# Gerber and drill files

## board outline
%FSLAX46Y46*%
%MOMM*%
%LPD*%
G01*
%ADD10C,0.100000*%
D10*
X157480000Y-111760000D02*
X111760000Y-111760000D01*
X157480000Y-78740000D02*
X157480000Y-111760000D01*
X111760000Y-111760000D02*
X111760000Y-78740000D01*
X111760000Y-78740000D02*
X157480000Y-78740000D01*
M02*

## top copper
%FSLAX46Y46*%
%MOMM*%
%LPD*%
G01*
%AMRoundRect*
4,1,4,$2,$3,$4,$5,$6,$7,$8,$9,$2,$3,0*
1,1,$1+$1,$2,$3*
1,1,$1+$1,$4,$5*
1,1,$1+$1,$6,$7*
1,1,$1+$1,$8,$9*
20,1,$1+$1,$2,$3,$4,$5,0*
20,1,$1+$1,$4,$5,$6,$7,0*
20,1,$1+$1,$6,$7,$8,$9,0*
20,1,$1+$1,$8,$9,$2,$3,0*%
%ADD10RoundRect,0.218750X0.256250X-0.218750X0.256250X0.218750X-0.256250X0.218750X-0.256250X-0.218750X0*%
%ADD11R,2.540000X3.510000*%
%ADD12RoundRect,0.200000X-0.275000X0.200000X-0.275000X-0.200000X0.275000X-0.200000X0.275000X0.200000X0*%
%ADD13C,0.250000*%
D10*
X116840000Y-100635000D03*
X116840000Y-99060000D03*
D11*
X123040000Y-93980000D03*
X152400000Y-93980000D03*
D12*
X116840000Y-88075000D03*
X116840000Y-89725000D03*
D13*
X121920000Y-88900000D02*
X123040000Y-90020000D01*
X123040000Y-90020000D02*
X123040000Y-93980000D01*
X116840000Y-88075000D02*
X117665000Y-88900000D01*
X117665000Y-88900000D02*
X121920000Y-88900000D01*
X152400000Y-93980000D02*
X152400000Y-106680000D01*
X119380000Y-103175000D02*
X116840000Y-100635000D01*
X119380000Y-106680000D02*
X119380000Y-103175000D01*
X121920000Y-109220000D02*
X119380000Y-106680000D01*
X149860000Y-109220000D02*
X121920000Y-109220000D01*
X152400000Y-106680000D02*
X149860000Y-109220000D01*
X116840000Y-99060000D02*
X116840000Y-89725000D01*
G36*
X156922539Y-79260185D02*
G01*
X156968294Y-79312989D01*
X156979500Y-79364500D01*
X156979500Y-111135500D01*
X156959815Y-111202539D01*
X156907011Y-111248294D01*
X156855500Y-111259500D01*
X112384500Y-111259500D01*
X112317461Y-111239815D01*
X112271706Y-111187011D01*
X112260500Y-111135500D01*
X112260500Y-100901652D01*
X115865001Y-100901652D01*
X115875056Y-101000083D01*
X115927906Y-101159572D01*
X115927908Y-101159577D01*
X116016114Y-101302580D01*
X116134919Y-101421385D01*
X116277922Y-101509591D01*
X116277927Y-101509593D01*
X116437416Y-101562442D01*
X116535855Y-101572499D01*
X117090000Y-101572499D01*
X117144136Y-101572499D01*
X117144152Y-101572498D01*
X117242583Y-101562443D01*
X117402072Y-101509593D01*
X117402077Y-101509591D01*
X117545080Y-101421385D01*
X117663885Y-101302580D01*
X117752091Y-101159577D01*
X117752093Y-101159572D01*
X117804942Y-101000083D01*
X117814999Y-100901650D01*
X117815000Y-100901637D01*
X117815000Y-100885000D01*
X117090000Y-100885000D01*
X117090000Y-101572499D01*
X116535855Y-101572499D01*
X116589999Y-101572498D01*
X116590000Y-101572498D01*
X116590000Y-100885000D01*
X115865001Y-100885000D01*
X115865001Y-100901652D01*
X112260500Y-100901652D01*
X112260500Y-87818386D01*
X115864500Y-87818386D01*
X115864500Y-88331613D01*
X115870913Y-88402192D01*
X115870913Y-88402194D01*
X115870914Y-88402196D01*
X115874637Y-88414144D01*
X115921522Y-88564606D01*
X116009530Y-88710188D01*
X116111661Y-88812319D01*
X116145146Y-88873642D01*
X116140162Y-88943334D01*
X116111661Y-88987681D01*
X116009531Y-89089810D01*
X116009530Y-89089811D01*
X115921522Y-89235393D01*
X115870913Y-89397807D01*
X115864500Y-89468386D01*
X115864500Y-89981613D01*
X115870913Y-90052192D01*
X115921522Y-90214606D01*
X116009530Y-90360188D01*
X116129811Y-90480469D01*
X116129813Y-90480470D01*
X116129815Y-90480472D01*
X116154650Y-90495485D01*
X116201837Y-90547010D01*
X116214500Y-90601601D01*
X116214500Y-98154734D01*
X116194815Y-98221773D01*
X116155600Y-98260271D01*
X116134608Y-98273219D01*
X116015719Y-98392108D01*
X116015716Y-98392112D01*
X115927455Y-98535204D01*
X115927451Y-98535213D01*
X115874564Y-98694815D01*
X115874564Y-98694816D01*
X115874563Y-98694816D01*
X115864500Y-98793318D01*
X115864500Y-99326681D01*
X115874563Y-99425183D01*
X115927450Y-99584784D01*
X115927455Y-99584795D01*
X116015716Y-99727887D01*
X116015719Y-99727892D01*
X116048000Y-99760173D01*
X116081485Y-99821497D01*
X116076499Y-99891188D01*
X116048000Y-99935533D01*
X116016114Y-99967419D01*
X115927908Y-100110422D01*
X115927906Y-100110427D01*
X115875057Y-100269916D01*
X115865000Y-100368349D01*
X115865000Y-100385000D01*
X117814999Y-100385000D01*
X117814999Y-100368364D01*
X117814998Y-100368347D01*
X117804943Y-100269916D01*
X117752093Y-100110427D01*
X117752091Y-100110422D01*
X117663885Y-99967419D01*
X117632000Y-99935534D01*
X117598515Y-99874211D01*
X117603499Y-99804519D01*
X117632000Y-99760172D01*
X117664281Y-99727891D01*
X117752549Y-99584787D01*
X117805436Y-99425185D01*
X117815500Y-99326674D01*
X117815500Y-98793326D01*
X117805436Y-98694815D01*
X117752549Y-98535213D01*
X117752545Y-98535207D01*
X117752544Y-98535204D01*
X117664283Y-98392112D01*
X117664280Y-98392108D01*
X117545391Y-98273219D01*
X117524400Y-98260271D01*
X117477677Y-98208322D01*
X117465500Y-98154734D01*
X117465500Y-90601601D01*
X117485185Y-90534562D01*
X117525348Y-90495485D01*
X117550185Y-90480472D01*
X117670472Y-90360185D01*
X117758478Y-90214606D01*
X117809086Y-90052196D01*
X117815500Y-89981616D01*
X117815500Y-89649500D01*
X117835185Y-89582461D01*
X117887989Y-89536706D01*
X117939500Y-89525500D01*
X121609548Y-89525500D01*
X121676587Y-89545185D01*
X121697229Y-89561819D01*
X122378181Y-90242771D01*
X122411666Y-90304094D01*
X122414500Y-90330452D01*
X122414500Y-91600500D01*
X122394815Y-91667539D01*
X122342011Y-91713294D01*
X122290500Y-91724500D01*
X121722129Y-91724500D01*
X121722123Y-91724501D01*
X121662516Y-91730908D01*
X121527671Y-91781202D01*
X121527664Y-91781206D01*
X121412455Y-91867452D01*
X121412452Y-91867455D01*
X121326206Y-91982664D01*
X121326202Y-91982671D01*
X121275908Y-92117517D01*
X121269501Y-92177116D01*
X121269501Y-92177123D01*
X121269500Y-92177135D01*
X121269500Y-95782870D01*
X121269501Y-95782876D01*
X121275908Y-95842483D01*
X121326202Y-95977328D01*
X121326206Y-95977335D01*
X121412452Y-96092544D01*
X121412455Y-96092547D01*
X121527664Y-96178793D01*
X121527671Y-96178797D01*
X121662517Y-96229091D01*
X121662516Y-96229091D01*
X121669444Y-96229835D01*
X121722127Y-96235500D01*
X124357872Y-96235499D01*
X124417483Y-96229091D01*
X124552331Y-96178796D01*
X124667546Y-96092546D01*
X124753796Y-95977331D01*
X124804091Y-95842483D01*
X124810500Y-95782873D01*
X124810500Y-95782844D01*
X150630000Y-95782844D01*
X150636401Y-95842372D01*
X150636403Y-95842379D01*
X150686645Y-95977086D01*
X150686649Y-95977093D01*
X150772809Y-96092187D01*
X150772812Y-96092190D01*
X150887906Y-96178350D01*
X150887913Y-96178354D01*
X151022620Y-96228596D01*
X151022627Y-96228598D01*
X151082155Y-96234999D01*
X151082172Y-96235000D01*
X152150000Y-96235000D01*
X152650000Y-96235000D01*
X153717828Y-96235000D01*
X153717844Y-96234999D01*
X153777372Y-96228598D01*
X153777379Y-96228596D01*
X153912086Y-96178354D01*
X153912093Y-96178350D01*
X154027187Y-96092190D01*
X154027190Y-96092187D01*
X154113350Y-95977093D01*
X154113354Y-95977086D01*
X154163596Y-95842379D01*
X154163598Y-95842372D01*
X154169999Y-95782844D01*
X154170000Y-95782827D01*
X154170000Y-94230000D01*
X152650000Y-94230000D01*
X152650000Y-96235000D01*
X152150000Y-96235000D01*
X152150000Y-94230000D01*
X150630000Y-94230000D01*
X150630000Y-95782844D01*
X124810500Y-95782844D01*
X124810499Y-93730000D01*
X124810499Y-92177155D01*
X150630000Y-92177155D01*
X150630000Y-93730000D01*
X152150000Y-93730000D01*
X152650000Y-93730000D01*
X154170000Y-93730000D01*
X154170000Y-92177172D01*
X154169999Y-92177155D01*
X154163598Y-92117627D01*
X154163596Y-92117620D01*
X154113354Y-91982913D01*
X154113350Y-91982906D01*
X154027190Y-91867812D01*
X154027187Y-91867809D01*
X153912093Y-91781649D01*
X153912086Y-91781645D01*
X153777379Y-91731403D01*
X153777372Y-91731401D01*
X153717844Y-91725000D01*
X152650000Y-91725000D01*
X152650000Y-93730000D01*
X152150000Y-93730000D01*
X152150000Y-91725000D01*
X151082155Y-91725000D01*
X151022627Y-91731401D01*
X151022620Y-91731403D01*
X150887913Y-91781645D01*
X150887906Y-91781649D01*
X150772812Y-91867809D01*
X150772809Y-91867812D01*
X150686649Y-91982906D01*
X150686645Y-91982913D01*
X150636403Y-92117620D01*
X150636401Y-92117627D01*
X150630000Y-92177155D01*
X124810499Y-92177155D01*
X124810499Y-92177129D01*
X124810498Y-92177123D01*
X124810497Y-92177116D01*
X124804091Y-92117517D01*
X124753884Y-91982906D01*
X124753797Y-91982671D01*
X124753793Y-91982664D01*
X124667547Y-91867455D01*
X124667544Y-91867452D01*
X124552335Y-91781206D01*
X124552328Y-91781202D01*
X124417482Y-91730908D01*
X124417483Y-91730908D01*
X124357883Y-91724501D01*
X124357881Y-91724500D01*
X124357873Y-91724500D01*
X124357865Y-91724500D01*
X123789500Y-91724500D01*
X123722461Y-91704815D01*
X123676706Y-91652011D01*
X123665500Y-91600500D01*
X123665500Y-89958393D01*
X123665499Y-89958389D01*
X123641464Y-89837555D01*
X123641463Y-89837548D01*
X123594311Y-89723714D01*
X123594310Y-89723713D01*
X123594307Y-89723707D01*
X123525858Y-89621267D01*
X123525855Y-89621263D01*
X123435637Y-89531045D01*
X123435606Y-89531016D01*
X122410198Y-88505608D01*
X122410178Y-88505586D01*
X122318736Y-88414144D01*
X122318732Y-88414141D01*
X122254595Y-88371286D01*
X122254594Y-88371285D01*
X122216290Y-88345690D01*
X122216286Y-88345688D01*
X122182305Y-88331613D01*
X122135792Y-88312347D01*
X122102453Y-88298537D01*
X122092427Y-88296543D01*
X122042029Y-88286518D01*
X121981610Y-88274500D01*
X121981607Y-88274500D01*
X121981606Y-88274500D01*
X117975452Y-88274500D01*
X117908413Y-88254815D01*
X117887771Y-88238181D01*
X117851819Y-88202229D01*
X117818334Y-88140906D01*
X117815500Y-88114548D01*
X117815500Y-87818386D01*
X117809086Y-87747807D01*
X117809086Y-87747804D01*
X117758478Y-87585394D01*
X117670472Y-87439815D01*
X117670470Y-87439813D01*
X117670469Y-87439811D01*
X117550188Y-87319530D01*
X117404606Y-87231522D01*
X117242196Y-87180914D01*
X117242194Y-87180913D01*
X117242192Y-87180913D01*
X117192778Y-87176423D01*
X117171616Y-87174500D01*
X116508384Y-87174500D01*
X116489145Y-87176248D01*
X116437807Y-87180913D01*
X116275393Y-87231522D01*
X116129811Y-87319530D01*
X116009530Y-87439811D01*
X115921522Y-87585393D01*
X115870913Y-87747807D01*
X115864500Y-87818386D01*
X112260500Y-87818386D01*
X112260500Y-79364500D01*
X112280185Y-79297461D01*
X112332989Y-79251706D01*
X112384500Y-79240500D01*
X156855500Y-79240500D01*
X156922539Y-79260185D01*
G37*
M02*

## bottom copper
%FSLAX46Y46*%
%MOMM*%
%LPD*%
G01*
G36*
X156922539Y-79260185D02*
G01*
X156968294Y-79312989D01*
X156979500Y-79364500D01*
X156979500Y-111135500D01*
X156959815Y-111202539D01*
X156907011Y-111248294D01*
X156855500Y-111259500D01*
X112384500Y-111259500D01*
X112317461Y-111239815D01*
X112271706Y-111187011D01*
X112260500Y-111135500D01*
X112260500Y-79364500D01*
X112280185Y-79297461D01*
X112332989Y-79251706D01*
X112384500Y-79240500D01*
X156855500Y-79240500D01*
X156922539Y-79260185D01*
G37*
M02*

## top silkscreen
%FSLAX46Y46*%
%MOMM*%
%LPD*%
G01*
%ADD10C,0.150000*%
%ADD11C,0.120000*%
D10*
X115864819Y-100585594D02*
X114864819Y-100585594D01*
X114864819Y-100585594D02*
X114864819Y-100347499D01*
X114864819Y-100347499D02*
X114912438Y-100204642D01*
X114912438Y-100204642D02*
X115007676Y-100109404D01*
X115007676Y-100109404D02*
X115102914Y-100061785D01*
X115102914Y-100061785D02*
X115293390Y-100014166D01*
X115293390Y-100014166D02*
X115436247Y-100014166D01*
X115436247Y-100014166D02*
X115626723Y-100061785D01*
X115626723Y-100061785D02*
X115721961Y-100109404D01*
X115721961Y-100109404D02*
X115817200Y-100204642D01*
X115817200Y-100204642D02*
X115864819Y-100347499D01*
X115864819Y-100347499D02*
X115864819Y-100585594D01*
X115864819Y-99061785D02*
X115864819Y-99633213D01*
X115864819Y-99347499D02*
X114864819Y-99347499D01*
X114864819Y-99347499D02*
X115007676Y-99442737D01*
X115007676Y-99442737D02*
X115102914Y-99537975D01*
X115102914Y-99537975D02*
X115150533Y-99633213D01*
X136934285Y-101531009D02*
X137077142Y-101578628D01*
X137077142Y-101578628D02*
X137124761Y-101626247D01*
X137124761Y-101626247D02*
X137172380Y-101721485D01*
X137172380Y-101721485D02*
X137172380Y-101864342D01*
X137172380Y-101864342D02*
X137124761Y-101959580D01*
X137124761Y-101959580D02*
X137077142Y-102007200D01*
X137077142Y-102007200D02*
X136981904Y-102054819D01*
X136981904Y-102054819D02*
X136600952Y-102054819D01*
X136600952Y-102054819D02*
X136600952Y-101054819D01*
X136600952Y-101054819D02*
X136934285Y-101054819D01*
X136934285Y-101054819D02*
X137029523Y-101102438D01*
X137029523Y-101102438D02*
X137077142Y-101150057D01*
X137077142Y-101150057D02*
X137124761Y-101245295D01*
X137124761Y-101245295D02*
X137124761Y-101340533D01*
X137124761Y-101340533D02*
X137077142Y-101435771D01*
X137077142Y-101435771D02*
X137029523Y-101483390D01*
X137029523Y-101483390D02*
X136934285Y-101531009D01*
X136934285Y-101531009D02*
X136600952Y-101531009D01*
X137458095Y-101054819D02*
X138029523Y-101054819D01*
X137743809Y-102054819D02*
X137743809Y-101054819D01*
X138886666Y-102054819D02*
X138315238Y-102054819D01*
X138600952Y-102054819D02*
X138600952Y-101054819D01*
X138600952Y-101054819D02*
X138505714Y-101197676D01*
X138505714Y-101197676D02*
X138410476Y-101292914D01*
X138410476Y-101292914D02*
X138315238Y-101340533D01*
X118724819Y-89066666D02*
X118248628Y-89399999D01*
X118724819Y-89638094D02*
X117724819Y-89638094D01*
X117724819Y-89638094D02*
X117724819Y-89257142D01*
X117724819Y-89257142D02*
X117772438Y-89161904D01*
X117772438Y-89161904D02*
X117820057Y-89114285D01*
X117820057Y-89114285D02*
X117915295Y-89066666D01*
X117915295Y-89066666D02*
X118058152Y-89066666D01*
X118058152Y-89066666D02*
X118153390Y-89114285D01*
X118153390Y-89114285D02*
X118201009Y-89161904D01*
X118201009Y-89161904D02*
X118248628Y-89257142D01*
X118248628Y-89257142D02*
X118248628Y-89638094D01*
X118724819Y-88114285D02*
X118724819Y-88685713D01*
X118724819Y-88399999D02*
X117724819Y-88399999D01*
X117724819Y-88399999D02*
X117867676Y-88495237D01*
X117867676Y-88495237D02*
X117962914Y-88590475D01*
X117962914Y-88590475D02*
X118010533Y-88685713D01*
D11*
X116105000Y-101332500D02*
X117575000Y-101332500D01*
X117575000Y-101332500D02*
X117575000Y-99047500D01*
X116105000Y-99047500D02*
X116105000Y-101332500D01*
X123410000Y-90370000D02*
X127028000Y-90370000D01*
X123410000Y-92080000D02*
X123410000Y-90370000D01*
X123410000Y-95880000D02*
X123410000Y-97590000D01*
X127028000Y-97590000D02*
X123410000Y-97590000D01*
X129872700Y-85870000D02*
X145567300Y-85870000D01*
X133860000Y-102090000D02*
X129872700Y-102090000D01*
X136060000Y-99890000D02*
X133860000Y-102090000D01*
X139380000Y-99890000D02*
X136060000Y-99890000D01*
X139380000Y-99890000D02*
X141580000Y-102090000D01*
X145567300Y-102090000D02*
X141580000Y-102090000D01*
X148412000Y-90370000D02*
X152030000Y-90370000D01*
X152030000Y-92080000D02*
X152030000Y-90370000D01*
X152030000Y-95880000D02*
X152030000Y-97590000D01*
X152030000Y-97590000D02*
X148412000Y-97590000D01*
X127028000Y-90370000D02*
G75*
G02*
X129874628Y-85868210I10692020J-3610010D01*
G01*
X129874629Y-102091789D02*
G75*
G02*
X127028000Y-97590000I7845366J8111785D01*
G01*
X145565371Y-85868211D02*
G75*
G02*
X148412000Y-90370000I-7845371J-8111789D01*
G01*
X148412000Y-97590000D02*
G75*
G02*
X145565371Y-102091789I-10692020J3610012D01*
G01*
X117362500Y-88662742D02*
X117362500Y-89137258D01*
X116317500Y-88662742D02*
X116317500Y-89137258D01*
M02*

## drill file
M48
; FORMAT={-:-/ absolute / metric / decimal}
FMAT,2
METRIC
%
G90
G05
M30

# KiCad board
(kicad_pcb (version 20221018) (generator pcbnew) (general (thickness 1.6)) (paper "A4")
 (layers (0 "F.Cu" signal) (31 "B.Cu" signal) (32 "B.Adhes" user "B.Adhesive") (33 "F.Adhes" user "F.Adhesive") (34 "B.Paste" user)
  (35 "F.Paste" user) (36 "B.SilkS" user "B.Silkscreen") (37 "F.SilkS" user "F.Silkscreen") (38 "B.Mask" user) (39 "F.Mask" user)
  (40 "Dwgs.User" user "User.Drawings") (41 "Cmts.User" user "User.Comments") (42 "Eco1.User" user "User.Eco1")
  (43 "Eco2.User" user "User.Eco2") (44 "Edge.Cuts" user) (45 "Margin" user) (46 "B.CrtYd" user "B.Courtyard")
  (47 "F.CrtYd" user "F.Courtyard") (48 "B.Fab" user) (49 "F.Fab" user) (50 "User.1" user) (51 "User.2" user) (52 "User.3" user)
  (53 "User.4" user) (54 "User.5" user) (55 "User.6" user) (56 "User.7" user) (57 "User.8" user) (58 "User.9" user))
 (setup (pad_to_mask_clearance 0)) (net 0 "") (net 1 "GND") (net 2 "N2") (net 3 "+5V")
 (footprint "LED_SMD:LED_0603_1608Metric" (layer "F.Cu") (at 116.84 99.8475 90)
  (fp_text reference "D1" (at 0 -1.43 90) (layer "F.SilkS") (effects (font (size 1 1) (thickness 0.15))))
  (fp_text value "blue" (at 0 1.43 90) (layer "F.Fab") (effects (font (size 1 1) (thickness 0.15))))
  (fp_line (start -1.485 -0.735) (end -1.485 0.735) (stroke (width 0.12) (type solid)) (layer "F.SilkS"))
  (fp_line (start -1.485 0.735) (end 0.8 0.735) (stroke (width 0.12) (type solid)) (layer "F.SilkS"))
  (fp_line (start 0.8 -0.735) (end -1.485 -0.735) (stroke (width 0.12) (type solid)) (layer "F.SilkS"))
  (pad "1" smd roundrect (at -0.7875 0 90) (size 0.875 0.95) (layers "F.Cu" "F.Paste" "F.Mask") (roundrect_rratio 0.25) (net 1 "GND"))
  (pad "2" smd roundrect (at 0.7875 0 90) (size 0.875 0.95) (layers "F.Cu" "F.Paste" "F.Mask") (roundrect_rratio 0.25) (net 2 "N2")))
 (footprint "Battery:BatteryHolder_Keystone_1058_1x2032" (layer "F.Cu") (at 137.72 93.98)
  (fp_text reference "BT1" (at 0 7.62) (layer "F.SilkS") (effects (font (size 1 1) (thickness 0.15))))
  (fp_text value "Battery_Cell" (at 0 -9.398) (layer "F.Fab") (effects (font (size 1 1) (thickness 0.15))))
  (fp_line (start -14.31 -3.61) (end -10.692 -3.61) (stroke (width 0.12) (type solid)) (layer "F.SilkS"))
  (fp_line (start -14.31 -1.9) (end -14.31 -3.61) (stroke (width 0.12) (type solid)) (layer "F.SilkS"))
  (fp_line (start -14.31 1.9) (end -14.31 3.61) (stroke (width 0.12) (type solid)) (layer "F.SilkS"))
  (fp_line (start -10.692 3.61) (end -14.31 3.61) (stroke (width 0.12) (type solid)) (layer "F.SilkS"))
  (fp_line (start -7.8473 -8.11) (end 7.8473 -8.11) (stroke (width 0.12) (type solid)) (layer "F.SilkS"))
  (fp_line (start -3.86 8.11) (end -7.8473 8.11) (stroke (width 0.12) (type solid)) (layer "F.SilkS"))
  (fp_line (start -1.66 5.91) (end -3.86 8.11) (stroke (width 0.12) (type solid)) (layer "F.SilkS"))
  (fp_line (start 1.66 5.91) (end -1.66 5.91) (stroke (width 0.12) (type solid)) (layer "F.SilkS"))
  (fp_line (start 1.66 5.91) (end 3.86 8.11) (stroke (width 0.12) (type solid)) (layer "F.SilkS"))
  (fp_line (start 7.8473 8.11) (end 3.86 8.11) (stroke (width 0.12) (type solid)) (layer "F.SilkS"))
  (fp_line (start 10.692 -3.61) (end 14.31 -3.61) (stroke (width 0.12) (type solid)) (layer "F.SilkS"))
  (fp_line (start 14.31 -1.9) (end 14.31 -3.61) (stroke (width 0.12) (type solid)) (layer "F.SilkS"))
  (fp_line (start 14.31 1.9) (end 14.31 3.61) (stroke (width 0.12) (type solid)) (layer "F.SilkS"))
  (fp_line (start 14.31 3.61) (end 10.692 3.61) (stroke (width 0.12) (type solid)) (layer "F.SilkS"))
  (fp_arc (start -10.692 -3.61) (mid -9.538084 -6.031244) (end -7.845371 -8.111789) (stroke (width 0.12) (type solid)) (layer "F.SilkS"))
  (fp_arc (start -7.845371 8.111789) (mid -9.538085 6.031244) (end -10.692 3.61) (stroke (width 0.12) (type solid)) (layer "F.SilkS"))
  (fp_arc (start 7.845371 -8.111789) (mid 9.538085 -6.031244) (end 10.692 -3.61) (stroke (width 0.12) (type solid)) (layer "F.SilkS"))
  (fp_arc (start 10.692 3.61) (mid 9.538084 6.031244) (end 7.845371 8.111789) (stroke (width 0.12) (type solid)) (layer "F.SilkS"))
  (pad "1" smd rect (at -14.68 0) (size 2.54 3.51) (layers "F.Cu" "F.Paste" "F.Mask") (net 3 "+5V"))
  (pad "2" smd rect (at 14.68 0) (size 2.54 3.51) (layers "F.Cu" "F.Paste" "F.Mask") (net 1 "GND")))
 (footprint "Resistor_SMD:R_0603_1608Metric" (layer "F.Cu") (at 116.84 88.9 -90)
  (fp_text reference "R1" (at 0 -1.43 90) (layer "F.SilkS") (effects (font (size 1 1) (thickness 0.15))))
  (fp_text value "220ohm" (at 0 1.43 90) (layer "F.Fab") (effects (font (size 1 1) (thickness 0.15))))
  (fp_line (start -0.237258 -0.5225) (end 0.237258 -0.5225) (stroke (width 0.12) (type solid)) (layer "F.SilkS"))
  (fp_line (start -0.237258 0.5225) (end 0.237258 0.5225) (stroke (width 0.12) (type solid)) (layer "F.SilkS"))
  (pad "1" smd roundrect (at -0.825 0 270) (size 0.8 0.95) (layers "F.Cu" "F.Paste" "F.Mask") (roundrect_rratio 0.25) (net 3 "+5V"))
  (pad "2" smd roundrect (at 0.825 0 270) (size 0.8 0.95) (layers "F.Cu" "F.Paste" "F.Mask") (roundrect_rratio 0.25) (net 2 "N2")))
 (gr_line (start 157.48 111.76) (end 111.76 111.76) (stroke (width 0.1) (type default)) (layer "Edge.Cuts"))
 (gr_line (start 157.48 78.74) (end 157.48 111.76) (stroke (width 0.1) (type default)) (layer "Edge.Cuts"))
 (gr_line (start 111.76 111.76) (end 111.76 78.74) (stroke (width 0.1) (type default)) (layer "Edge.Cuts"))
 (gr_line (start 111.76 78.74) (end 157.48 78.74) (stroke (width 0.1) (type default)) (layer "Edge.Cuts"))
 (segment (start 121.92 88.9) (end 123.04 90.02) (width 0.25) (layer "F.Cu") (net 3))
 (segment (start 123.04 90.02) (end 123.04 93.98) (width 0.25) (layer "F.Cu") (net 3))
 (segment (start 116.84 88.075) (end 117.665 88.9) (width 0.25) (layer "F.Cu") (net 3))
 (segment (start 117.665 88.9) (end 121.92 88.9) (width 0.25) (layer "F.Cu") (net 3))
 (segment (start 152.4 93.98) (end 152.4 106.68) (width 0.25) (layer "F.Cu") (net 1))
 (segment (start 119.38 103.175) (end 116.84 100.635) (width 0.25) (layer "F.Cu") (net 1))
 (segment (start 119.38 106.68) (end 119.38 103.175) (width 0.25) (layer "F.Cu") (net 1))
 (segment (start 121.92 109.22) (end 119.38 106.68) (width 0.25) (layer "F.Cu") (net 1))
 (segment (start 149.86 109.22) (end 121.92 109.22) (width 0.25) (layer "F.Cu") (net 1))
 (segment (start 152.4 106.68) (end 149.86 109.22) (width 0.25) (layer "F.Cu") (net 1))
 (segment (start 116.84 99.06) (end 116.84 89.725) (width 0.25) (layer "F.Cu") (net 2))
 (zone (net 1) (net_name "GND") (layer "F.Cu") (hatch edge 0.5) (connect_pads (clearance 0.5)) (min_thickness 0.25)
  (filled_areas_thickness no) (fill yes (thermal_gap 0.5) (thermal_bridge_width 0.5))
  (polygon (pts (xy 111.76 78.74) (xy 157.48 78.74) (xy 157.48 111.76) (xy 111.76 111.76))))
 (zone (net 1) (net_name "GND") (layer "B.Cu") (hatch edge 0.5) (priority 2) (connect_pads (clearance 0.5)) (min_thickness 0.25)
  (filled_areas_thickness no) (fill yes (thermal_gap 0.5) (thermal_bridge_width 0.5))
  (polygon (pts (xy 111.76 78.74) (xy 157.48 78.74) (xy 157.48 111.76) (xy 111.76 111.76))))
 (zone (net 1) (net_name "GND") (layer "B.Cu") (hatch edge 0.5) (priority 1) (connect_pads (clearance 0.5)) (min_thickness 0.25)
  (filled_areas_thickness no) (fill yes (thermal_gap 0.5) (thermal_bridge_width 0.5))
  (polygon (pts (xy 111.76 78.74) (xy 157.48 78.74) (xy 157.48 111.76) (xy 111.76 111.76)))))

